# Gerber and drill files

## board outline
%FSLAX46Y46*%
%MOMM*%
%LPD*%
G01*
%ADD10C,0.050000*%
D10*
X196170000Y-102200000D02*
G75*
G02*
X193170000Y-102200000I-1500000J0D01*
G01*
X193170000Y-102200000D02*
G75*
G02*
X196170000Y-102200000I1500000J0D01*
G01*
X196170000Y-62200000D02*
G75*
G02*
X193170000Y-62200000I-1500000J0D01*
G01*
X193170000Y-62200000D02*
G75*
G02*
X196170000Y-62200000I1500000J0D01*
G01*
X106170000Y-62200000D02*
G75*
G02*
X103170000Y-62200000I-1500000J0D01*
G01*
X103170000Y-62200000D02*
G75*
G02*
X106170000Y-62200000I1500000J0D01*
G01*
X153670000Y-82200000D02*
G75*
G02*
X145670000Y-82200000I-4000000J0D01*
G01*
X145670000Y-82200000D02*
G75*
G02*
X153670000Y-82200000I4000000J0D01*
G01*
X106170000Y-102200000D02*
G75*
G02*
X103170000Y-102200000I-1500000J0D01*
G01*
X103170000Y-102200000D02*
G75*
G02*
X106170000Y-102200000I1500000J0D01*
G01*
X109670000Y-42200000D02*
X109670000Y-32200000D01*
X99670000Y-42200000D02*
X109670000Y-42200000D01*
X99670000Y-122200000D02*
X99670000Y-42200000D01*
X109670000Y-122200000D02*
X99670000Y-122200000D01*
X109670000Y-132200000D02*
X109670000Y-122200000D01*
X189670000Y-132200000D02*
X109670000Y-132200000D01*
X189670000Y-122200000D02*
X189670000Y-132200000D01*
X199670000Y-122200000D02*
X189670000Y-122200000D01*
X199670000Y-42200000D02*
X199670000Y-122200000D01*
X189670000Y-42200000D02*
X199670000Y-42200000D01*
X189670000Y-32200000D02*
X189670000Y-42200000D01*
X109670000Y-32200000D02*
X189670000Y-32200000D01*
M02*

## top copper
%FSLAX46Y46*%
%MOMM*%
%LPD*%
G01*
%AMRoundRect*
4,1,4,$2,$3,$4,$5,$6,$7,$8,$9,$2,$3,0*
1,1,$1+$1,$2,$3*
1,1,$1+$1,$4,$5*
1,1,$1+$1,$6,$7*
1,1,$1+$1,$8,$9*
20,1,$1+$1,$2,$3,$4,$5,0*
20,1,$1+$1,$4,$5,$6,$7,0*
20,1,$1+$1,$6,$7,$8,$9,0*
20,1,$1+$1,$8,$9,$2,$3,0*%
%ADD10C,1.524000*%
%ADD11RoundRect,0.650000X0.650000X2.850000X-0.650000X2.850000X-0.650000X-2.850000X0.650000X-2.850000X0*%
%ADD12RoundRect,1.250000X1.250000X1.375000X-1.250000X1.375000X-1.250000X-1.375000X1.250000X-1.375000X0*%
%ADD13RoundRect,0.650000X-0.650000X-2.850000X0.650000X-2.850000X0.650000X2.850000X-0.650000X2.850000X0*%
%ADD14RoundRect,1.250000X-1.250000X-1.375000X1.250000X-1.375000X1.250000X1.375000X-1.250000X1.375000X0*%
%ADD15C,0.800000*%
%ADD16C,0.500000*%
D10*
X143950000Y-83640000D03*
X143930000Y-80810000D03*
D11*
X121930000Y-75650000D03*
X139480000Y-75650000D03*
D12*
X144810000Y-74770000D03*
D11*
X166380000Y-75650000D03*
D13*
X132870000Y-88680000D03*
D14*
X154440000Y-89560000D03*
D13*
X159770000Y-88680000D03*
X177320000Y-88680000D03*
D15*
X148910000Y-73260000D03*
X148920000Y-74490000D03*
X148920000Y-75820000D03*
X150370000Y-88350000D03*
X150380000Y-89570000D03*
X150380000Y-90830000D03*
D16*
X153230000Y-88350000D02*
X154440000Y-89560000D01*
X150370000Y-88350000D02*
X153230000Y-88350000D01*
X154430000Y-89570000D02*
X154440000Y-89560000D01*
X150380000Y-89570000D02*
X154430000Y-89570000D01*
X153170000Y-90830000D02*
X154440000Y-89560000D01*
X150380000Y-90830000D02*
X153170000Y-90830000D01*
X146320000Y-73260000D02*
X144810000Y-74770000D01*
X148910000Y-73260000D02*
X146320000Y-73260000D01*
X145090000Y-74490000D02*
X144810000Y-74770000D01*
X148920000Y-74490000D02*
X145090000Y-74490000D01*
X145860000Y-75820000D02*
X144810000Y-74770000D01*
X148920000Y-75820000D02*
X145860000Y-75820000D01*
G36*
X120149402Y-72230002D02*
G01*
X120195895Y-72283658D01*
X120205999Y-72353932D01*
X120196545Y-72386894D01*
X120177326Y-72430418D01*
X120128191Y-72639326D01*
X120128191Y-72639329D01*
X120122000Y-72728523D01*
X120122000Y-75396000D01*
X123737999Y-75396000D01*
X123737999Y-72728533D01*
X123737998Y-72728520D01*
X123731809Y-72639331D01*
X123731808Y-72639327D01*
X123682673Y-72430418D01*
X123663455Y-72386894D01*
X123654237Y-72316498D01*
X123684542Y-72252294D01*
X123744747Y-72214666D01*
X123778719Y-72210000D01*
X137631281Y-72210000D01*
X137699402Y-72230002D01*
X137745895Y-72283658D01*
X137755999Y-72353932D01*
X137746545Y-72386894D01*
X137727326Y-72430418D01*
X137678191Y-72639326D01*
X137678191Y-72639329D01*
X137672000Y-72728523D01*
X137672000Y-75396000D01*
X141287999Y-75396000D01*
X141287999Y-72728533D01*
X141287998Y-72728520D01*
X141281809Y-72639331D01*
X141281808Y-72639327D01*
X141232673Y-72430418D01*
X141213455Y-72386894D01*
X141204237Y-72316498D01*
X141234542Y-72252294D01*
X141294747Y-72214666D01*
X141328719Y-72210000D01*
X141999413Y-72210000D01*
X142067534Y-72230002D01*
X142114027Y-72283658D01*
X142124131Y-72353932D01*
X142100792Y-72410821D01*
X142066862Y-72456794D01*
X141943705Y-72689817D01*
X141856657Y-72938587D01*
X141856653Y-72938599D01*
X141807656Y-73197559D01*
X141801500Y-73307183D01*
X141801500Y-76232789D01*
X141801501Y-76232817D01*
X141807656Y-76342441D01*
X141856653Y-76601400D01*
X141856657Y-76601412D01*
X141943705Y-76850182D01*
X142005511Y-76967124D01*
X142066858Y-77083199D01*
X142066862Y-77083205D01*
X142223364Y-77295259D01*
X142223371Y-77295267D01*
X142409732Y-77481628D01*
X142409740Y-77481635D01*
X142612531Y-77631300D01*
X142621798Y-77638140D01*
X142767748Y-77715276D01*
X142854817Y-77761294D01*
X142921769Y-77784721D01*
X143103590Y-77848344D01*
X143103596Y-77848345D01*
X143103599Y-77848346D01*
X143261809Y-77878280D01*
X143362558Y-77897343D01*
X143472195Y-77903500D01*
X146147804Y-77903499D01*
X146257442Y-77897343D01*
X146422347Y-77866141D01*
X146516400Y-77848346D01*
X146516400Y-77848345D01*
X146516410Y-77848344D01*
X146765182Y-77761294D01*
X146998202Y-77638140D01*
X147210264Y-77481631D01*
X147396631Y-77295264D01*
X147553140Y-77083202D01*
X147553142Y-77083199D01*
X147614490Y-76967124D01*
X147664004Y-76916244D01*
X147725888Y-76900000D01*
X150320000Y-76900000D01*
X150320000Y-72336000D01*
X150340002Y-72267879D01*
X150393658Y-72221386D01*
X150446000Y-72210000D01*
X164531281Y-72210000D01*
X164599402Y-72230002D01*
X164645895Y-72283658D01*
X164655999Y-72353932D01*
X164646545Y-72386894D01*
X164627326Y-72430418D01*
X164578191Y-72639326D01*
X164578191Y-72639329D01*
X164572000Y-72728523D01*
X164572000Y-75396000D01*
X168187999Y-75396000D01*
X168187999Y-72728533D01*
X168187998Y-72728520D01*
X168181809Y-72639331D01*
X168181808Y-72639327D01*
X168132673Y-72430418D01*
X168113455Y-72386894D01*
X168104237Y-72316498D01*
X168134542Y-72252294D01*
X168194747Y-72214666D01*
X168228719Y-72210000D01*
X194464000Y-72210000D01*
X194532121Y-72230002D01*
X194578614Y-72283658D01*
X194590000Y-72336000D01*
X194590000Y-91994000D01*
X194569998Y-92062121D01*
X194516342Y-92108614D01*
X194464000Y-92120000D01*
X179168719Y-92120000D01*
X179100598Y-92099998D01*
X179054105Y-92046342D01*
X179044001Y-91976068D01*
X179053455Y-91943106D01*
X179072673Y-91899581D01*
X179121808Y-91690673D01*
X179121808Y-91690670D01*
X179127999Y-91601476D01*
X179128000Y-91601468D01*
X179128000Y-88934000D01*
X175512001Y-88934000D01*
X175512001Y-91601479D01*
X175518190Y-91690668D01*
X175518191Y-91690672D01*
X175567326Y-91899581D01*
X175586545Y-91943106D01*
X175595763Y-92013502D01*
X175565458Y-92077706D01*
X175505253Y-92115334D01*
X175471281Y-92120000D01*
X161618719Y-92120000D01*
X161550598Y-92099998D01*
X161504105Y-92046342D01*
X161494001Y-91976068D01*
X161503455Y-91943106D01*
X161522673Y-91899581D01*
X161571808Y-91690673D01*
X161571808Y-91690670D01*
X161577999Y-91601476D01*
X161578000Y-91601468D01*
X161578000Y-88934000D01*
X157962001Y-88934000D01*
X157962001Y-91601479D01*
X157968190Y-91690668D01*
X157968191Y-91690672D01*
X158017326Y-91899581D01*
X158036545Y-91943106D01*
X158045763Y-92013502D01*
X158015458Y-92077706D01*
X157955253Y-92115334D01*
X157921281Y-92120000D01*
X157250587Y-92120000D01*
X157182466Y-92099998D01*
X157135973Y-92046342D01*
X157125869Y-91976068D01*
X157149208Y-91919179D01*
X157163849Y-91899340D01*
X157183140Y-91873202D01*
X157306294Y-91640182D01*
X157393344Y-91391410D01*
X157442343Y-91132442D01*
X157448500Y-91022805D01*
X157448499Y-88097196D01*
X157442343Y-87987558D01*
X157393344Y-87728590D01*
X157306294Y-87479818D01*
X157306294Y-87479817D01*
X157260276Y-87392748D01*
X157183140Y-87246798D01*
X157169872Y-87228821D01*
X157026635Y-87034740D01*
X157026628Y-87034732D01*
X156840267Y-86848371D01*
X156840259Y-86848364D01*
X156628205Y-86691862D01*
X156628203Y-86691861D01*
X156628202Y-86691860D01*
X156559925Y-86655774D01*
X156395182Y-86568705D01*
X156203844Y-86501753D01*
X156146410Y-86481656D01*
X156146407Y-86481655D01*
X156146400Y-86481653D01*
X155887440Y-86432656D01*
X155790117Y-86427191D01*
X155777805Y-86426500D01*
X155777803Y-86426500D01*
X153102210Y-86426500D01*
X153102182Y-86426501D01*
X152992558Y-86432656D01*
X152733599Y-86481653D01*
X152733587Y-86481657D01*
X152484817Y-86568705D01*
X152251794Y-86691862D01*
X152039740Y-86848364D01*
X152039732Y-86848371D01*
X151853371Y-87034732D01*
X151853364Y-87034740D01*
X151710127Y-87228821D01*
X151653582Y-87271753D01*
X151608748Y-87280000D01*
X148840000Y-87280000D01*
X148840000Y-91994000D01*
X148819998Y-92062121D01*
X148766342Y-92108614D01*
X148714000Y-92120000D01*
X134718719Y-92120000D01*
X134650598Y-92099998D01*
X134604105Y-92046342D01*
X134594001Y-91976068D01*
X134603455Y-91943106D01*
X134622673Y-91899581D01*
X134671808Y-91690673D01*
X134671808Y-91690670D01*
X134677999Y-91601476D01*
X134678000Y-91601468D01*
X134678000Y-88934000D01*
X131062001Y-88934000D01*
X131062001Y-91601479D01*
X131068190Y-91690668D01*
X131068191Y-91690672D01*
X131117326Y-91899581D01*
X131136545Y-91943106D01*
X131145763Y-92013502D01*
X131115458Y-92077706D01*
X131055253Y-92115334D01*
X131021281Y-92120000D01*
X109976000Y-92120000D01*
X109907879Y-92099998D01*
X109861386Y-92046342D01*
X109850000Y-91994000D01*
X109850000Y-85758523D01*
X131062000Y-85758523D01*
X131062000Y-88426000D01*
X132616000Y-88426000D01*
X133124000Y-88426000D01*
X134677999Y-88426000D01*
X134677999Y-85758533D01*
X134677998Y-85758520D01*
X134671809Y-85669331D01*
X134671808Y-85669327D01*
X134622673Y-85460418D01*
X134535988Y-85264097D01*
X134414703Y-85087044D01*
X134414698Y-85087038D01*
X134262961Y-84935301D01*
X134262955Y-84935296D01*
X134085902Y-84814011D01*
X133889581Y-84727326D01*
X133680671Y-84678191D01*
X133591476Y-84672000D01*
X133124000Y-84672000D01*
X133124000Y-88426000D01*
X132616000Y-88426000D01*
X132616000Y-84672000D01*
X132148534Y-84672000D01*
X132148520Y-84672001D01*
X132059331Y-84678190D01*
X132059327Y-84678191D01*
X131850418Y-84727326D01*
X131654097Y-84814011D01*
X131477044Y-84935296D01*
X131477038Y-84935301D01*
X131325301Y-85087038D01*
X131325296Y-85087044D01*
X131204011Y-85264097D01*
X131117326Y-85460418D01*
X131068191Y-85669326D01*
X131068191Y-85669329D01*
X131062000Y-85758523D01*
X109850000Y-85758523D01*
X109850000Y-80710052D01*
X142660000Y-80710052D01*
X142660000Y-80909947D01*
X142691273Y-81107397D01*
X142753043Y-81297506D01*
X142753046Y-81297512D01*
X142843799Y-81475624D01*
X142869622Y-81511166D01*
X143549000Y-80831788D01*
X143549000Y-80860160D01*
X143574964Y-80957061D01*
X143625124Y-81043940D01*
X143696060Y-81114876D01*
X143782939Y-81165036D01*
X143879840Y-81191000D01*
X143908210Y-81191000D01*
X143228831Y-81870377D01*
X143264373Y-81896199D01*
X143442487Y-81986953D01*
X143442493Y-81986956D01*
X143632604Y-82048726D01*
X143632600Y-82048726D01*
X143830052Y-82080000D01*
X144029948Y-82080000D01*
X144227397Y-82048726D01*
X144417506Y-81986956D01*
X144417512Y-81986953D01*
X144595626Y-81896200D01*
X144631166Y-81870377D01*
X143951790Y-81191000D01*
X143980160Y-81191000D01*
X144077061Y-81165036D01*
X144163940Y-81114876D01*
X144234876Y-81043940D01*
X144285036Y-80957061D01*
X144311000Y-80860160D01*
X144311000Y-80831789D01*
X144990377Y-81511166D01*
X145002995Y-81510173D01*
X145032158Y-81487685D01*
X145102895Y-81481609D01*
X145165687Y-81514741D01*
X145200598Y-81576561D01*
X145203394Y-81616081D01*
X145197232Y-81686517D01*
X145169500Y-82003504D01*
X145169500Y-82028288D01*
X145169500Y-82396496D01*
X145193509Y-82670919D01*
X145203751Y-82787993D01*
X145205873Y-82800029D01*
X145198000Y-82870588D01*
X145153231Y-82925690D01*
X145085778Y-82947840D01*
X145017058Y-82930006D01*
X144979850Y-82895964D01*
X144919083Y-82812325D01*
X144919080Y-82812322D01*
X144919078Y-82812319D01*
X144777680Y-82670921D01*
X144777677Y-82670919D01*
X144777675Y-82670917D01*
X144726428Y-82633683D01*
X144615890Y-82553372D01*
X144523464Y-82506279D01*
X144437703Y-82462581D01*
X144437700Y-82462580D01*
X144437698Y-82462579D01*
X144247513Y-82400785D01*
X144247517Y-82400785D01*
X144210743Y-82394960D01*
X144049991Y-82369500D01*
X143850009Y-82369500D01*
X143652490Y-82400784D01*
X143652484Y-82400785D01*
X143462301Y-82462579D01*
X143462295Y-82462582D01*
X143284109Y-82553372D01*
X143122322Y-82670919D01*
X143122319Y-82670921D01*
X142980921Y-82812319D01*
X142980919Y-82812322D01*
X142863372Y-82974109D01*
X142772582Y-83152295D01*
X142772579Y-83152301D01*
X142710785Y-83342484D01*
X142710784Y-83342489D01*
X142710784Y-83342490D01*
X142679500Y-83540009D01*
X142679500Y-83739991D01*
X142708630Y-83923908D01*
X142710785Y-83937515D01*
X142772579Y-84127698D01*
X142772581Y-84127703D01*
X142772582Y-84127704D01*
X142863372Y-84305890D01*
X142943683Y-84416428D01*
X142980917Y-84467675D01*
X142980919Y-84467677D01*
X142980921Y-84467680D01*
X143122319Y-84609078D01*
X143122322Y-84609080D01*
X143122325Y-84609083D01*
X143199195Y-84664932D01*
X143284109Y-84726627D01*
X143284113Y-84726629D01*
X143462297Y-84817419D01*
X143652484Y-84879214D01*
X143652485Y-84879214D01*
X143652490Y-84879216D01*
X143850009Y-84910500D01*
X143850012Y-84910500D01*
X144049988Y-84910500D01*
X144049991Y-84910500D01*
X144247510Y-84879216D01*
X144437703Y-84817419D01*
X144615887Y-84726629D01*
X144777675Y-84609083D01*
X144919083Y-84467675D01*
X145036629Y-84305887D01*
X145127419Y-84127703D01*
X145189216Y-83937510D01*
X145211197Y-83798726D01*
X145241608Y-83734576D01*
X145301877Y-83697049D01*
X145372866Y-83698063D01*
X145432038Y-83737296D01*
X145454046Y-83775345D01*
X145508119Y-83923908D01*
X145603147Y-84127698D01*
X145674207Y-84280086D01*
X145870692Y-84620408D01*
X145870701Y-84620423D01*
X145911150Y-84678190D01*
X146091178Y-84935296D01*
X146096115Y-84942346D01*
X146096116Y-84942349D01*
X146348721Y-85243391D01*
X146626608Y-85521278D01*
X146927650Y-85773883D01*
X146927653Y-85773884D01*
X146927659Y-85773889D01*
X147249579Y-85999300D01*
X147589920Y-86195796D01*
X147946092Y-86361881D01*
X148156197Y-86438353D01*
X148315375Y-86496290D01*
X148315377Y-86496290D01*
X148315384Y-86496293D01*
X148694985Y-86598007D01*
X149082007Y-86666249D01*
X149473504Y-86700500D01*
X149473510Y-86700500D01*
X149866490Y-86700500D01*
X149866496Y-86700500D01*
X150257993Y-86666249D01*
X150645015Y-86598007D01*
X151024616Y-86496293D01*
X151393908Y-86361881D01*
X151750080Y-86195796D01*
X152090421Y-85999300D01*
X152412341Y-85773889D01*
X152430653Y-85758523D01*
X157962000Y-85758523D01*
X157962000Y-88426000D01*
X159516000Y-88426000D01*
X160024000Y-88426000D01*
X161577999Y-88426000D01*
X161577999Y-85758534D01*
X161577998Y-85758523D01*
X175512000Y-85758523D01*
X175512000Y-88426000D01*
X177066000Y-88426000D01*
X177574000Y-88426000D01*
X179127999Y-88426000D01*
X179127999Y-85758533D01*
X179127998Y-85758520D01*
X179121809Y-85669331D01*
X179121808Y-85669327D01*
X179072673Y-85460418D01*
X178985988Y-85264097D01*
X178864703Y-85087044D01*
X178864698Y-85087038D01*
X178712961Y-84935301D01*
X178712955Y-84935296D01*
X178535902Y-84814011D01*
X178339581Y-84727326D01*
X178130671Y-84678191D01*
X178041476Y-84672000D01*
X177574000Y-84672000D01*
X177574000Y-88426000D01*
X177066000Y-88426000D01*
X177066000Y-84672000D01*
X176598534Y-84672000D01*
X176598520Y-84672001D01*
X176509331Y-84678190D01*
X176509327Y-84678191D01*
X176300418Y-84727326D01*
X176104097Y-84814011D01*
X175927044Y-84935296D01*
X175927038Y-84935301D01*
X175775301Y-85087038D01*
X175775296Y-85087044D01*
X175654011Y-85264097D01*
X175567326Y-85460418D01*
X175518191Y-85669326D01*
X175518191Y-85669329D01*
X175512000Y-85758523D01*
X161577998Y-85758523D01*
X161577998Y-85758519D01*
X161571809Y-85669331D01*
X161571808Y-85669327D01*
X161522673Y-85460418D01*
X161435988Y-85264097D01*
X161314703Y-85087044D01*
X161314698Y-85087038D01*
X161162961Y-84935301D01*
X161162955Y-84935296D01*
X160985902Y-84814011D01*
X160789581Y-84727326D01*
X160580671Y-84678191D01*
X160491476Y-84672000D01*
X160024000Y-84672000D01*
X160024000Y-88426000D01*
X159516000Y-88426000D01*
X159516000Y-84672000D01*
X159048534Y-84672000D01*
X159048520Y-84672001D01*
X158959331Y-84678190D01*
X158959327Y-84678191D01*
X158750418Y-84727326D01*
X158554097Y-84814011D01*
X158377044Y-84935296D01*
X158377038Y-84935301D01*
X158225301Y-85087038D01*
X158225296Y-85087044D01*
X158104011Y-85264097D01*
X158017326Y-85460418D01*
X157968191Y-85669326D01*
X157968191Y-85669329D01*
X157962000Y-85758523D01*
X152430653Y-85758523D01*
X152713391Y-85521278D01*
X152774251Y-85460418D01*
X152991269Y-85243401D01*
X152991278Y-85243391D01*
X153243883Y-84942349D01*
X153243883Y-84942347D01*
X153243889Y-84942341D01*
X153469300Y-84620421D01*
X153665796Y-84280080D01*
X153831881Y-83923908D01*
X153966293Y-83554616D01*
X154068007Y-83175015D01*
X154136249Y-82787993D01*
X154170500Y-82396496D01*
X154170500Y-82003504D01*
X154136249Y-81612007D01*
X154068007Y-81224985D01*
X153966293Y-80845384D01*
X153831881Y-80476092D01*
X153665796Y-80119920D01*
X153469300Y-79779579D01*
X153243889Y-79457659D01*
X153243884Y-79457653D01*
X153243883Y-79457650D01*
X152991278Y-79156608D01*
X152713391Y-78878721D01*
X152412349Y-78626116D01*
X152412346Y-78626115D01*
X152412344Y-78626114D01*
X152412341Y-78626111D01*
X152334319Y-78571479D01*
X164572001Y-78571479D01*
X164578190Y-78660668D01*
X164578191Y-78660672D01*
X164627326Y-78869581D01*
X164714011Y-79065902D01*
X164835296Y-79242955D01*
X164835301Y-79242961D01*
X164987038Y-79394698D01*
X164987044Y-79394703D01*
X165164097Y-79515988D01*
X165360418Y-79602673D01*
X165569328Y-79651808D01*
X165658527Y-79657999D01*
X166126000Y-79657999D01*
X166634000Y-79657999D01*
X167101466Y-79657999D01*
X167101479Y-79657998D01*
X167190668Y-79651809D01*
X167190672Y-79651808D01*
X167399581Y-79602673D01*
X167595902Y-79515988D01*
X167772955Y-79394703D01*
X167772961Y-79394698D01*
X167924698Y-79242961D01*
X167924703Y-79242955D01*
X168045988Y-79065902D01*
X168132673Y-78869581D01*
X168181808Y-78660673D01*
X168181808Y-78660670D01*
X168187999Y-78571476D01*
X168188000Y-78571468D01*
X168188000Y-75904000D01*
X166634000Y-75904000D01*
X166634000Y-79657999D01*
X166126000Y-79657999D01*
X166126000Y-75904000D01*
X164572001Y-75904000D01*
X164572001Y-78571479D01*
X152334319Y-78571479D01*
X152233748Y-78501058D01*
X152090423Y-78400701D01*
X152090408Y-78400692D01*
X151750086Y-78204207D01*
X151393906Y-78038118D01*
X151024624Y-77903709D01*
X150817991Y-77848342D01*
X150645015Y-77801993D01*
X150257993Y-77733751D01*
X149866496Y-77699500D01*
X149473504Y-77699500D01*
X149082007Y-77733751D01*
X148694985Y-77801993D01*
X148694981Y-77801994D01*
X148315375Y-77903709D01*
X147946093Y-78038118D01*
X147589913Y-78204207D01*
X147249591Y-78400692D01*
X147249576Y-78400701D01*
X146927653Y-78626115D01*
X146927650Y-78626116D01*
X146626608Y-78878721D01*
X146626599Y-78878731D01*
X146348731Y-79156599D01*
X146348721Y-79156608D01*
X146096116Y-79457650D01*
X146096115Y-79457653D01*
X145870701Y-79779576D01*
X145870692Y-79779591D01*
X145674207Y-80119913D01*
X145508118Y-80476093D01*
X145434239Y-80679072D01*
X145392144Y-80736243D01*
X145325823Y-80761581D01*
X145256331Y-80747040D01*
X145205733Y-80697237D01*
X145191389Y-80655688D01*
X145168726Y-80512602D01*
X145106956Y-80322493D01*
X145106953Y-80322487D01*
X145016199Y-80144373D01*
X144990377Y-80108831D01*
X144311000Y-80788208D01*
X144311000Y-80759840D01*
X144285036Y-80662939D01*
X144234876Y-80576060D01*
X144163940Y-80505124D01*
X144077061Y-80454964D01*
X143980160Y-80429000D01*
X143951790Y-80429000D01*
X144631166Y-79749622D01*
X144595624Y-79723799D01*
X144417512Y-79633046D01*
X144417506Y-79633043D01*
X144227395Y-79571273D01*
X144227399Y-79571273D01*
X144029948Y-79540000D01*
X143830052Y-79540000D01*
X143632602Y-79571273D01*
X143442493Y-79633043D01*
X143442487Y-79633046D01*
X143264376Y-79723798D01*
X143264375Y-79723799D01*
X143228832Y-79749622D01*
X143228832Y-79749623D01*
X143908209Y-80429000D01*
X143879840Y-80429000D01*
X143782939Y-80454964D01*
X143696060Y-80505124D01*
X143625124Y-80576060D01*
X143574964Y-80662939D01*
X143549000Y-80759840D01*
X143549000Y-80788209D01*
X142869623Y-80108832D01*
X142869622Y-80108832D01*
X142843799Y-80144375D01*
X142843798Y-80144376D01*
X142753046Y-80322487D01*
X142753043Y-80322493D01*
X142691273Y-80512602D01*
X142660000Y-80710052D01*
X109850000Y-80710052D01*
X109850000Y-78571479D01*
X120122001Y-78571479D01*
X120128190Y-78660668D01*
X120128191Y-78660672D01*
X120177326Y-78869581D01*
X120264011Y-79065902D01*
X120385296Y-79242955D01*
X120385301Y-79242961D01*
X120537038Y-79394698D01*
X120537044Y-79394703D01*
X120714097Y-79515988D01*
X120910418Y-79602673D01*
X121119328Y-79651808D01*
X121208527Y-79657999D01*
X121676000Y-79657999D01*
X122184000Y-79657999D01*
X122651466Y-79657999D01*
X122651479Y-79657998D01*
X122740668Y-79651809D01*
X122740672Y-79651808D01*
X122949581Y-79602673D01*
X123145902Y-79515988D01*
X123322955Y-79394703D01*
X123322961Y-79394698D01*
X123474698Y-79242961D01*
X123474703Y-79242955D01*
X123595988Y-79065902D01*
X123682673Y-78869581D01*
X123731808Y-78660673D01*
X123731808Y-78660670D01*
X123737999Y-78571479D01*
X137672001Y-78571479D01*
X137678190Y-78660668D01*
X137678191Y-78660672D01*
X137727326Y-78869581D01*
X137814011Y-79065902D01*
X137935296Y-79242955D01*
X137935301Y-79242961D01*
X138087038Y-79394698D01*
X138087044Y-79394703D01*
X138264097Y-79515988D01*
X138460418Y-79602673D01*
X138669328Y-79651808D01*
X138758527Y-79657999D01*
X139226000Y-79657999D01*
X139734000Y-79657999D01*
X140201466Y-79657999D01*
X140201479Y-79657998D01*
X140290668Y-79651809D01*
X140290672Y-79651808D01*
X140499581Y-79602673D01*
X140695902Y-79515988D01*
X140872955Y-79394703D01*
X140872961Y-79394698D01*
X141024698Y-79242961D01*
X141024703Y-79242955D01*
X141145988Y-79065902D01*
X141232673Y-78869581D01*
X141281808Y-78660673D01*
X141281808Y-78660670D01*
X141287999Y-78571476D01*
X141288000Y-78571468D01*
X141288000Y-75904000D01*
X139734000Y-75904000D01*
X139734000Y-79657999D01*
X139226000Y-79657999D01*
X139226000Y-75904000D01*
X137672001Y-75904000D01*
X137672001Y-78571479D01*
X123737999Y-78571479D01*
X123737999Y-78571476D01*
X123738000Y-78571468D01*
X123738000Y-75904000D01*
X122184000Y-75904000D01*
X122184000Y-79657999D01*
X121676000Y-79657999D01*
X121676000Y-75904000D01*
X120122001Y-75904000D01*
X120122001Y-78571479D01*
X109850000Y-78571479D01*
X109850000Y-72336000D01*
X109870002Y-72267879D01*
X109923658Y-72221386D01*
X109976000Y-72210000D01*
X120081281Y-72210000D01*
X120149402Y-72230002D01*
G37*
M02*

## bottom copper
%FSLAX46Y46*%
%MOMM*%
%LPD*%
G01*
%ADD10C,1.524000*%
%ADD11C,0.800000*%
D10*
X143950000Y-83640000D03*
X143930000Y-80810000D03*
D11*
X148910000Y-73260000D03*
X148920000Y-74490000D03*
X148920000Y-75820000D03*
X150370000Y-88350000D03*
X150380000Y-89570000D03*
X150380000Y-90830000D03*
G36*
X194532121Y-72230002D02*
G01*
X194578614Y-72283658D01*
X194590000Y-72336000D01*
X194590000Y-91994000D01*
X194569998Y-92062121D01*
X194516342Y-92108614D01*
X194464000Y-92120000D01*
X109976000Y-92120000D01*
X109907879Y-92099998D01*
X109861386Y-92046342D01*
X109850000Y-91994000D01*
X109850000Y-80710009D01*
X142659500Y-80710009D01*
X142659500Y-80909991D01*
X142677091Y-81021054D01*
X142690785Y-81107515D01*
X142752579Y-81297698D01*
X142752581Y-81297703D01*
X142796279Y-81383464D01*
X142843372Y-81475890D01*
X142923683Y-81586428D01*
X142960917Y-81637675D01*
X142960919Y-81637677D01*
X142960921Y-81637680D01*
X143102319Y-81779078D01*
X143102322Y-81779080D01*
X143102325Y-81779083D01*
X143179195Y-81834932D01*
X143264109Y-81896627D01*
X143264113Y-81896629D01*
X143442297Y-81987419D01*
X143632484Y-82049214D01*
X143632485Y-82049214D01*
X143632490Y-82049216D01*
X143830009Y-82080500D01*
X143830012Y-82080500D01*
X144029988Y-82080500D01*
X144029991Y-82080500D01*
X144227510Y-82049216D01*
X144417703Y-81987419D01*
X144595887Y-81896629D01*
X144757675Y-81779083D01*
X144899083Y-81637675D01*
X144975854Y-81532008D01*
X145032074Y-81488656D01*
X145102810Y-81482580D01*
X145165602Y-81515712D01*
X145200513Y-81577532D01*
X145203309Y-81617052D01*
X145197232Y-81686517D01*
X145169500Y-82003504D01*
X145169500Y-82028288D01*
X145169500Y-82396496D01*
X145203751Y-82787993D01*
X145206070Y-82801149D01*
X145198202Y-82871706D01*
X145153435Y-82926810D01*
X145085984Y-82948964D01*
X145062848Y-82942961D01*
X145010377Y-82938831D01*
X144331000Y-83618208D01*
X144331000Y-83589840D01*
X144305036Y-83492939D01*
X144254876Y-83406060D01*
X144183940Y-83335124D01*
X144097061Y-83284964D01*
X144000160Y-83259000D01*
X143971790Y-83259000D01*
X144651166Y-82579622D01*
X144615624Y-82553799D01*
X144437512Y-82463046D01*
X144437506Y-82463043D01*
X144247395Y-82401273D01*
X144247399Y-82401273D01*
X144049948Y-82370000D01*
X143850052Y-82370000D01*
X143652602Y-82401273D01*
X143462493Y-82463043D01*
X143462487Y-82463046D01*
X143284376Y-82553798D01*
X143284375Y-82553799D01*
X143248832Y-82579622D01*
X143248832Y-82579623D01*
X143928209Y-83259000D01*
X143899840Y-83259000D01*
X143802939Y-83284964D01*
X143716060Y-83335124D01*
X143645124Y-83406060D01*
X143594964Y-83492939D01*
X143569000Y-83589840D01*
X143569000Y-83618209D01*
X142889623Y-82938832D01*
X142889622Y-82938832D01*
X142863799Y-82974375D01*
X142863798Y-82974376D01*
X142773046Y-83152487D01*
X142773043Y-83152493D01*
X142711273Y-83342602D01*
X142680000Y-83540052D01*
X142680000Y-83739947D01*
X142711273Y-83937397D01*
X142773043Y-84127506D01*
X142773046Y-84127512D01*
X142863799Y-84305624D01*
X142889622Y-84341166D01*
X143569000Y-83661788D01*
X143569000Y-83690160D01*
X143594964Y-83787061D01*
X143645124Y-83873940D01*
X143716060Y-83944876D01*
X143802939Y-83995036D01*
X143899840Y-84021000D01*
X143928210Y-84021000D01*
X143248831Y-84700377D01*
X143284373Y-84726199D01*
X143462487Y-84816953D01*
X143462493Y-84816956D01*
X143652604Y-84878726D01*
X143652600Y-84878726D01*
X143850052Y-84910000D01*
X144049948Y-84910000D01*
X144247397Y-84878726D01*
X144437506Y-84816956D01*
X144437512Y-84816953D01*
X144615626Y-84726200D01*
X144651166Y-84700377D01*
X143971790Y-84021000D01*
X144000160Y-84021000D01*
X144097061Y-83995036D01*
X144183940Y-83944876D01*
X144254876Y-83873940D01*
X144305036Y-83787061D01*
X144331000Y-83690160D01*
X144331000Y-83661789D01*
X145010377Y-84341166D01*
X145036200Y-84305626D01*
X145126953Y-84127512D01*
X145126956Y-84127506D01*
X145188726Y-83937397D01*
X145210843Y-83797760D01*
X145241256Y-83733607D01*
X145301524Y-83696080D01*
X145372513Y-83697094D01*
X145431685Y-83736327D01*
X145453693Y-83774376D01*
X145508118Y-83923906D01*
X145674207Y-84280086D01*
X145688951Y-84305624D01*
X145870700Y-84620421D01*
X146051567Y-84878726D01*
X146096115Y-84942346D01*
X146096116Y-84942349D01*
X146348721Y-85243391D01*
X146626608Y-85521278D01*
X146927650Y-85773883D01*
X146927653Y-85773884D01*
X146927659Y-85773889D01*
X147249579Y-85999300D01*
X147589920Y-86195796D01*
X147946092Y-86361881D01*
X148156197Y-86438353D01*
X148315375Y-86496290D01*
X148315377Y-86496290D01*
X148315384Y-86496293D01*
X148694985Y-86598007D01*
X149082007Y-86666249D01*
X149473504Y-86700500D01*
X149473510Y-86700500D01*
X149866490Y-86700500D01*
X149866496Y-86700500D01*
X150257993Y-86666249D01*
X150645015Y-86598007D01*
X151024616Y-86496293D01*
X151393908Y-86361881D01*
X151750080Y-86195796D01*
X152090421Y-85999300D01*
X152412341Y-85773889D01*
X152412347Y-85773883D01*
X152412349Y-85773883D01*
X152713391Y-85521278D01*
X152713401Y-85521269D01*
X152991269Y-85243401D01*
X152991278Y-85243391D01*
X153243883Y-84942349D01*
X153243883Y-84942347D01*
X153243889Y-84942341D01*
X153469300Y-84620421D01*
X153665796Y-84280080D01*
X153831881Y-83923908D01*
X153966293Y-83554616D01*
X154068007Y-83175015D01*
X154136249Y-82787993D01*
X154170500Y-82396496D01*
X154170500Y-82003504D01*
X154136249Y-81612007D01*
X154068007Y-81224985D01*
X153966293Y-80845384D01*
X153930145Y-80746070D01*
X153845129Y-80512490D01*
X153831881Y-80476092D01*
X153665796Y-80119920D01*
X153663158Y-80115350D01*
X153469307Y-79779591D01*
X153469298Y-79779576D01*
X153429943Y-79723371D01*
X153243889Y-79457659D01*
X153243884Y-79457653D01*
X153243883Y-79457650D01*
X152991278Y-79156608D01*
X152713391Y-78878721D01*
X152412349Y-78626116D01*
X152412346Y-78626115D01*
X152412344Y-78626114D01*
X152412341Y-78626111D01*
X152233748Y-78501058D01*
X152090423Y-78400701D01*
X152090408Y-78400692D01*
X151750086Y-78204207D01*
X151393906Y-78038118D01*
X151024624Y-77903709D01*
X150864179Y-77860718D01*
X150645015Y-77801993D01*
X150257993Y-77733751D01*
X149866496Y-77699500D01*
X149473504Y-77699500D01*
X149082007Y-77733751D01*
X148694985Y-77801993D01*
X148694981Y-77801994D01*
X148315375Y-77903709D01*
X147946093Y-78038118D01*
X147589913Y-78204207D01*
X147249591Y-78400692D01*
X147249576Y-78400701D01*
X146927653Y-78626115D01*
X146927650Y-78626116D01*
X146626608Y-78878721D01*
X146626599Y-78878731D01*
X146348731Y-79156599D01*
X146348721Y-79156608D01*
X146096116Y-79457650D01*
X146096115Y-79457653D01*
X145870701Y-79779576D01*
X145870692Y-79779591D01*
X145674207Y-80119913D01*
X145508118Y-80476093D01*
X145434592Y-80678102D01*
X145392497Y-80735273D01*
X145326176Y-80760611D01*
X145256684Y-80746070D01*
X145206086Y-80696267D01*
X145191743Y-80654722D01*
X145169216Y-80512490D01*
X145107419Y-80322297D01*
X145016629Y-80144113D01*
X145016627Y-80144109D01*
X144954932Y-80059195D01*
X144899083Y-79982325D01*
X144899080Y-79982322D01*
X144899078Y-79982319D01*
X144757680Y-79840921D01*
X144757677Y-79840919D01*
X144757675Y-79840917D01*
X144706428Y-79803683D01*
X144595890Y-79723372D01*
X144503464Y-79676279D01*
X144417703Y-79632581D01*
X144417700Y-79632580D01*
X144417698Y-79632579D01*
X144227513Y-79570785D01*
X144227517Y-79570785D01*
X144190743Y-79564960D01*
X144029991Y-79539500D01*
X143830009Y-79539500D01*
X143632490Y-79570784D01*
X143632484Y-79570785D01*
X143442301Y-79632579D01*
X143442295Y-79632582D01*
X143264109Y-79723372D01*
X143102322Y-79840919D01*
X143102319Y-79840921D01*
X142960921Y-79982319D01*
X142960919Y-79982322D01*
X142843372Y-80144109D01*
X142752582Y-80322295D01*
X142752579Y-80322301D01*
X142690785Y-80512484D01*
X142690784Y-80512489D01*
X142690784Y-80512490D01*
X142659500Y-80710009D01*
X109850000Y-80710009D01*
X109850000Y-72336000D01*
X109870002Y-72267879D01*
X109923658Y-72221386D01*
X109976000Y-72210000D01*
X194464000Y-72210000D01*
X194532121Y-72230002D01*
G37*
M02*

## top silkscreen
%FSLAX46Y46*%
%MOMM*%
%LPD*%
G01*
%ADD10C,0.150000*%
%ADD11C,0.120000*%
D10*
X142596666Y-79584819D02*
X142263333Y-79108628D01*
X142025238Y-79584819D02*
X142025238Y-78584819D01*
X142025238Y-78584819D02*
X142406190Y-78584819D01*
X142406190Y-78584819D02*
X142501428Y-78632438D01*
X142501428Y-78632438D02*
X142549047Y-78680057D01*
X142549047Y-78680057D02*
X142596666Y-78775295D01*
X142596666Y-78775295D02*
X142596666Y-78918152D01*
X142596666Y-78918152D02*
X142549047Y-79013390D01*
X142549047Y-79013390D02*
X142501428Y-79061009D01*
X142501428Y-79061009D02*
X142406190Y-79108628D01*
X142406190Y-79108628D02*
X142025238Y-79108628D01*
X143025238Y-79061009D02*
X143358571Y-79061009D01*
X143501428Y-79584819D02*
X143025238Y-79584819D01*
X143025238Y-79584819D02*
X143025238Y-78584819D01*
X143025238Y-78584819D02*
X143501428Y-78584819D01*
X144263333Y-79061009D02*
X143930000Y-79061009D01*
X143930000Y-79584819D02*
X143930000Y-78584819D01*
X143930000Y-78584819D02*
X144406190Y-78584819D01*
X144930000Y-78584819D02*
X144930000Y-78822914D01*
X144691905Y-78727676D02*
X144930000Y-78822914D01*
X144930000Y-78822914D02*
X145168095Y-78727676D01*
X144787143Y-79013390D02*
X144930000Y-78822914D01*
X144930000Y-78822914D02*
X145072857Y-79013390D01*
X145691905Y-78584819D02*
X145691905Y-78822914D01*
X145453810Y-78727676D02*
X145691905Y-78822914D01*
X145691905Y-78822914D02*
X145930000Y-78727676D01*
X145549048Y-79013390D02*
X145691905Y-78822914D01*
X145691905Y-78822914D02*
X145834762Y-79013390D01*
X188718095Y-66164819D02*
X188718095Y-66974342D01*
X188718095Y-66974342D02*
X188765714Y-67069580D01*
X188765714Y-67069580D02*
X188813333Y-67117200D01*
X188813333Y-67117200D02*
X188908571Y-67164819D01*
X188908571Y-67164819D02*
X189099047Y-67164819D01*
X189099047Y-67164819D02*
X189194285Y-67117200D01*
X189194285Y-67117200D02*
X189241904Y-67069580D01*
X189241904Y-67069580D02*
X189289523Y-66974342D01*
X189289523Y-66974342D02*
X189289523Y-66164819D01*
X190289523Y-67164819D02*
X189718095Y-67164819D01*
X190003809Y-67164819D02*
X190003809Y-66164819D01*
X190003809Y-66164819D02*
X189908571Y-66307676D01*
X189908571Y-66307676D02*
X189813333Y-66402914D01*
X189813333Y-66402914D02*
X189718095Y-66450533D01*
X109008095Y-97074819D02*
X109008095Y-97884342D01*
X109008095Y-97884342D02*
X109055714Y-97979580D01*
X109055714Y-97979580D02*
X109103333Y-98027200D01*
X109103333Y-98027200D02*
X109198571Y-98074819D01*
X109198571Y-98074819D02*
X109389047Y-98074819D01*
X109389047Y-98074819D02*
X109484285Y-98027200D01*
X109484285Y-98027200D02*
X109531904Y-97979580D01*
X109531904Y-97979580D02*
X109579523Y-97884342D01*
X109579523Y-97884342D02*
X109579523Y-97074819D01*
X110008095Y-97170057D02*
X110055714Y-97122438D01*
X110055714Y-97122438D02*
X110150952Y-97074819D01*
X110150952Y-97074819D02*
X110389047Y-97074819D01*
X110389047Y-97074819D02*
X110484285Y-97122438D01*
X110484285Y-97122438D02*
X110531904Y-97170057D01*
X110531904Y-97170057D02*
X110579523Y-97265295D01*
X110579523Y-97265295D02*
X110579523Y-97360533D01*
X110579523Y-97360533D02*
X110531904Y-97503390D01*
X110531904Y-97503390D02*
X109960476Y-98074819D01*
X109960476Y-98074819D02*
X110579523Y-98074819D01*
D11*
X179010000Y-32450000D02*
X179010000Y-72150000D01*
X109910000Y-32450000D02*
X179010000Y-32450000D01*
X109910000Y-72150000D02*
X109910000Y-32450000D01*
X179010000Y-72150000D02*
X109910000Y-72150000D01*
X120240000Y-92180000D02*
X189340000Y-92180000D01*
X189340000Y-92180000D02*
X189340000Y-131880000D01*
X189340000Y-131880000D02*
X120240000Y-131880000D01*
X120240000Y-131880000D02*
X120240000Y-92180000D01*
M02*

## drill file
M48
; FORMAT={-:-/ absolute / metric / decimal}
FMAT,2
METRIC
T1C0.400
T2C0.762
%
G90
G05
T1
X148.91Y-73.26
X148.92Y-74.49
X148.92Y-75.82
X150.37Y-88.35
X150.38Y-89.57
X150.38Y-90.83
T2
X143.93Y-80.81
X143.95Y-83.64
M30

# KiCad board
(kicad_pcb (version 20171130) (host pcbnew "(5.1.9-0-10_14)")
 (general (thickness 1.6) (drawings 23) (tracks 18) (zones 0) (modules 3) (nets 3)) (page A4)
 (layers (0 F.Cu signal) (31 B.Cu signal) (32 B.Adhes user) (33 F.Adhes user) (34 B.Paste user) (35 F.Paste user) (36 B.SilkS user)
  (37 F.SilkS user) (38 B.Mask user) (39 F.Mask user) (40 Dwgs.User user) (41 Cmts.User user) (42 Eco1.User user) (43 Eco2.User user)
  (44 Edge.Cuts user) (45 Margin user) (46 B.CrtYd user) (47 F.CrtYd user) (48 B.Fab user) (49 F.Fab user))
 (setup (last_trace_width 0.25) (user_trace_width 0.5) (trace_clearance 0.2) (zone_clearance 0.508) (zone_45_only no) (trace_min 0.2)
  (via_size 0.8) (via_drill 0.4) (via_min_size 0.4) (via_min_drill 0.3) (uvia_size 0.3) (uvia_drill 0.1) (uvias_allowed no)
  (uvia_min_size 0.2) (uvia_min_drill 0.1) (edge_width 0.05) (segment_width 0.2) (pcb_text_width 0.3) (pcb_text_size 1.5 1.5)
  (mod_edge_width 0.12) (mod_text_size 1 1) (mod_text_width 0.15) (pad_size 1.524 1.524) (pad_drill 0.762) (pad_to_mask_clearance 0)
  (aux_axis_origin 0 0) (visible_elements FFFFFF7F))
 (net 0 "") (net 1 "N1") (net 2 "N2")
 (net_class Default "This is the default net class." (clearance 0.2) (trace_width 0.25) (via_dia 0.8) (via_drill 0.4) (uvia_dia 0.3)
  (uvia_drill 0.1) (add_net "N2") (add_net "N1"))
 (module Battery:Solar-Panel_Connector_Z (layer F.Cu) (at 143.93 78.63)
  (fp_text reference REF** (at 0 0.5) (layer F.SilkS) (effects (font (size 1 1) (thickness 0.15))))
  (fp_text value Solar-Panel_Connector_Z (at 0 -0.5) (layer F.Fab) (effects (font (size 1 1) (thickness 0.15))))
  (pad 2 thru_hole circle (at 0.02 5.01) (size 1.524 1.524) (drill 0.762) (layers *.Cu *.Mask) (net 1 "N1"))
  (pad 1 thru_hole circle (at 0 2.18) (size 1.524 1.524) (drill 0.762) (layers *.Cu *.Mask) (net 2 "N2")))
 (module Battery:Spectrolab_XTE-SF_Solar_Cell (layer F.Cu) (at 179.01 72.15 180)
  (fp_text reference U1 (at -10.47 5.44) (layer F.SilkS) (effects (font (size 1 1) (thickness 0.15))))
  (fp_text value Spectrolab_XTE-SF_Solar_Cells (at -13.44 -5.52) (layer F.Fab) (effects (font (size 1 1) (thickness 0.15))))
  (fp_line (start 0 39.7) (end 0 0) (layer F.SilkS) (width 0.12))
  (fp_line (start 69.1 39.7) (end 0 39.7) (layer F.SilkS) (width 0.12))
  (fp_line (start 69.1 0) (end 69.1 39.7) (layer F.SilkS) (width 0.12))
  (fp_line (start 0 0) (end 69.1 0) (layer F.SilkS) (width 0.12))
  (pad 4 smd roundrect (at 57.08 -3.5 180) (size 2.6 7) (layers F.Cu F.Paste F.Mask) (roundrect_rratio 0.25) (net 2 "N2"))
  (pad 3 smd roundrect (at 39.53 -3.5 180) (size 2.6 7) (layers F.Cu F.Paste F.Mask) (roundrect_rratio 0.25) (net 2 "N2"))
  (pad 2 smd roundrect (at 34.2 -2.62 180) (size 5 5.25) (layers F.Cu F.Paste F.Mask) (roundrect_rratio 0.25) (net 1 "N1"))
  (pad 1 smd roundrect (at 12.63 -3.5 180) (size 2.6 7) (layers F.Cu F.Paste F.Mask) (roundrect_rratio 0.25) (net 2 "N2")))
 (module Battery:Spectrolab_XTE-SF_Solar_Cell (layer F.Cu) (at 120.24 92.18)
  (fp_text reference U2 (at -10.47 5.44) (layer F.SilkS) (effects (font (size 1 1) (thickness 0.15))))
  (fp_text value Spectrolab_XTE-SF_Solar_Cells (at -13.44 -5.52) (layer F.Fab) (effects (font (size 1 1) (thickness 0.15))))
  (fp_line (start 0 0) (end 69.1 0) (layer F.SilkS) (width 0.12))
  (fp_line (start 69.1 0) (end 69.1 39.7) (layer F.SilkS) (width 0.12))
  (fp_line (start 69.1 39.7) (end 0 39.7) (layer F.SilkS) (width 0.12))
  (fp_line (start 0 39.7) (end 0 0) (layer F.SilkS) (width 0.12))
  (pad 1 smd roundrect (at 12.63 -3.5) (size 2.6 7) (layers F.Cu F.Paste F.Mask) (roundrect_rratio 0.25) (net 2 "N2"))
  (pad 2 smd roundrect (at 34.2 -2.62) (size 5 5.25) (layers F.Cu F.Paste F.Mask) (roundrect_rratio 0.25) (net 1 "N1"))
  (pad 3 smd roundrect (at 39.53 -3.5) (size 2.6 7) (layers F.Cu F.Paste F.Mask) (roundrect_rratio 0.25) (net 2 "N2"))
  (pad 4 smd roundrect (at 57.08 -3.5) (size 2.6 7) (layers F.Cu F.Paste F.Mask) (roundrect_rratio 0.25) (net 2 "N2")))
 (gr_circle (center 194.67 102.2) (end 196.17 102.2) (layer Edge.Cuts) (width 0.05))
 (gr_circle (center 194.67 62.2) (end 196.17 62.2) (layer Edge.Cuts) (width 0.05))
 (gr_circle (center 104.67 62.2) (end 106.17 62.2) (layer Edge.Cuts) (width 0.05))
 (gr_circle (center 149.67 82.2) (end 153.67 82.2) (layer Edge.Cuts) (width 0.05))
 (gr_circle (center 104.67 102.2) (end 106.17 102.2) (layer Edge.Cuts) (width 0.05))
 (gr_line (start 109.67 42.2) (end 109.67 32.2) (layer Edge.Cuts) (width 0.05))
 (gr_line (start 99.67 42.2) (end 109.67 42.2) (layer Edge.Cuts) (width 0.05))
 (gr_line (start 99.67 122.2) (end 99.67 42.2) (layer Edge.Cuts) (width 0.05))
 (gr_line (start 109.67 122.2) (end 99.67 122.2) (layer Edge.Cuts) (width 0.05))
 (gr_line (start 109.67 132.2) (end 109.67 122.2) (layer Edge.Cuts) (width 0.05))
 (gr_line (start 189.67 132.2) (end 109.67 132.2) (layer Edge.Cuts) (width 0.05))
 (gr_line (start 189.67 122.2) (end 189.67 132.2) (layer Edge.Cuts) (width 0.05))
 (gr_line (start 199.67 122.2) (end 189.67 122.2) (layer Edge.Cuts) (width 0.05))
 (gr_line (start 199.67 42.2) (end 199.67 122.2) (layer Edge.Cuts) (width 0.05))
 (gr_line (start 189.67 42.2) (end 199.67 42.2) (layer Edge.Cuts) (width 0.05))
 (gr_line (start 189.67 32.2) (end 189.67 42.2) (layer Edge.Cuts) (width 0.05))
 (gr_line (start 109.67 32.2) (end 189.67 32.2) (layer Edge.Cuts) (width 0.05))
 (via (at 148.91 73.26) (size 0.8) (drill 0.4) (layers F.Cu B.Cu) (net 1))
 (via (at 148.92 74.49) (size 0.8) (drill 0.4) (layers F.Cu B.Cu) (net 1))
 (via (at 148.92 75.82) (size 0.8) (drill 0.4) (layers F.Cu B.Cu) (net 1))
 (via (at 150.37 88.35) (size 0.8) (drill 0.4) (layers F.Cu B.Cu) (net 1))
 (via (at 150.38 89.57) (size 0.8) (drill 0.4) (layers F.Cu B.Cu) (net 1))
 (via (at 150.38 90.83) (size 0.8) (drill 0.4) (layers F.Cu B.Cu) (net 1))
 (segment (start 153.23 88.35) (end 154.44 89.56) (width 0.5) (layer F.Cu) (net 1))
 (segment (start 150.37 88.35) (end 153.23 88.35) (width 0.5) (layer F.Cu) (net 1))
 (segment (start 154.43 89.57) (end 154.44 89.56) (width 0.5) (layer F.Cu) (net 1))
 (segment (start 150.38 89.57) (end 154.43 89.57) (width 0.5) (layer F.Cu) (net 1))
 (segment (start 153.17 90.83) (end 154.44 89.56) (width 0.5) (layer F.Cu) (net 1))
 (segment (start 150.38 90.83) (end 153.17 90.83) (width 0.5) (layer F.Cu) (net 1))
 (segment (start 146.32 73.26) (end 144.81 74.77) (width 0.5) (layer F.Cu) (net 1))
 (segment (start 148.91 73.26) (end 146.32 73.26) (width 0.5) (layer F.Cu) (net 1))
 (segment (start 145.09 74.49) (end 144.81 74.77) (width 0.5) (layer F.Cu) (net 1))
 (segment (start 148.92 74.49) (end 145.09 74.49) (width 0.5) (layer F.Cu) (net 1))
 (segment (start 145.86 75.82) (end 144.81 74.77) (width 0.5) (layer F.Cu) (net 1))
 (segment (start 148.92 75.82) (end 145.86 75.82) (width 0.5) (layer F.Cu) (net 1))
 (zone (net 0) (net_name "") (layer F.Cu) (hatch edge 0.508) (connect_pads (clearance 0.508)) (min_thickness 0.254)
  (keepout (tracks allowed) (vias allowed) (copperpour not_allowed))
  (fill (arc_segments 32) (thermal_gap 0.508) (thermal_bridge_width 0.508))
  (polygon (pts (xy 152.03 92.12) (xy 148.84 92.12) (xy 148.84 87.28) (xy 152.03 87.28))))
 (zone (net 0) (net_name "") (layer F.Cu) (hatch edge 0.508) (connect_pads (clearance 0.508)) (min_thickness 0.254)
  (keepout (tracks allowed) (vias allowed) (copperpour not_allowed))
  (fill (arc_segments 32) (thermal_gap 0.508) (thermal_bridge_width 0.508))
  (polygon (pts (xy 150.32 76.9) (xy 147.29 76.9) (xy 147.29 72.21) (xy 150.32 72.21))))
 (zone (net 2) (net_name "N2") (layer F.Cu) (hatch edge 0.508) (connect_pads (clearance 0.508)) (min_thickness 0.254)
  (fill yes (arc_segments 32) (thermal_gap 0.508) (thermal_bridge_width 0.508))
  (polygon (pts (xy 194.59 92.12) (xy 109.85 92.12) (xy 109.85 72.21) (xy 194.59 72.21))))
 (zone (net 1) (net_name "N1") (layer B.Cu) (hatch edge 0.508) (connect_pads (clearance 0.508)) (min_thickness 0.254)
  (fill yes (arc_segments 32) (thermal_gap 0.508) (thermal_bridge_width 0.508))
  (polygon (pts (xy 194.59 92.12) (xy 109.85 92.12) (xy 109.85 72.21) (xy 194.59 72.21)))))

